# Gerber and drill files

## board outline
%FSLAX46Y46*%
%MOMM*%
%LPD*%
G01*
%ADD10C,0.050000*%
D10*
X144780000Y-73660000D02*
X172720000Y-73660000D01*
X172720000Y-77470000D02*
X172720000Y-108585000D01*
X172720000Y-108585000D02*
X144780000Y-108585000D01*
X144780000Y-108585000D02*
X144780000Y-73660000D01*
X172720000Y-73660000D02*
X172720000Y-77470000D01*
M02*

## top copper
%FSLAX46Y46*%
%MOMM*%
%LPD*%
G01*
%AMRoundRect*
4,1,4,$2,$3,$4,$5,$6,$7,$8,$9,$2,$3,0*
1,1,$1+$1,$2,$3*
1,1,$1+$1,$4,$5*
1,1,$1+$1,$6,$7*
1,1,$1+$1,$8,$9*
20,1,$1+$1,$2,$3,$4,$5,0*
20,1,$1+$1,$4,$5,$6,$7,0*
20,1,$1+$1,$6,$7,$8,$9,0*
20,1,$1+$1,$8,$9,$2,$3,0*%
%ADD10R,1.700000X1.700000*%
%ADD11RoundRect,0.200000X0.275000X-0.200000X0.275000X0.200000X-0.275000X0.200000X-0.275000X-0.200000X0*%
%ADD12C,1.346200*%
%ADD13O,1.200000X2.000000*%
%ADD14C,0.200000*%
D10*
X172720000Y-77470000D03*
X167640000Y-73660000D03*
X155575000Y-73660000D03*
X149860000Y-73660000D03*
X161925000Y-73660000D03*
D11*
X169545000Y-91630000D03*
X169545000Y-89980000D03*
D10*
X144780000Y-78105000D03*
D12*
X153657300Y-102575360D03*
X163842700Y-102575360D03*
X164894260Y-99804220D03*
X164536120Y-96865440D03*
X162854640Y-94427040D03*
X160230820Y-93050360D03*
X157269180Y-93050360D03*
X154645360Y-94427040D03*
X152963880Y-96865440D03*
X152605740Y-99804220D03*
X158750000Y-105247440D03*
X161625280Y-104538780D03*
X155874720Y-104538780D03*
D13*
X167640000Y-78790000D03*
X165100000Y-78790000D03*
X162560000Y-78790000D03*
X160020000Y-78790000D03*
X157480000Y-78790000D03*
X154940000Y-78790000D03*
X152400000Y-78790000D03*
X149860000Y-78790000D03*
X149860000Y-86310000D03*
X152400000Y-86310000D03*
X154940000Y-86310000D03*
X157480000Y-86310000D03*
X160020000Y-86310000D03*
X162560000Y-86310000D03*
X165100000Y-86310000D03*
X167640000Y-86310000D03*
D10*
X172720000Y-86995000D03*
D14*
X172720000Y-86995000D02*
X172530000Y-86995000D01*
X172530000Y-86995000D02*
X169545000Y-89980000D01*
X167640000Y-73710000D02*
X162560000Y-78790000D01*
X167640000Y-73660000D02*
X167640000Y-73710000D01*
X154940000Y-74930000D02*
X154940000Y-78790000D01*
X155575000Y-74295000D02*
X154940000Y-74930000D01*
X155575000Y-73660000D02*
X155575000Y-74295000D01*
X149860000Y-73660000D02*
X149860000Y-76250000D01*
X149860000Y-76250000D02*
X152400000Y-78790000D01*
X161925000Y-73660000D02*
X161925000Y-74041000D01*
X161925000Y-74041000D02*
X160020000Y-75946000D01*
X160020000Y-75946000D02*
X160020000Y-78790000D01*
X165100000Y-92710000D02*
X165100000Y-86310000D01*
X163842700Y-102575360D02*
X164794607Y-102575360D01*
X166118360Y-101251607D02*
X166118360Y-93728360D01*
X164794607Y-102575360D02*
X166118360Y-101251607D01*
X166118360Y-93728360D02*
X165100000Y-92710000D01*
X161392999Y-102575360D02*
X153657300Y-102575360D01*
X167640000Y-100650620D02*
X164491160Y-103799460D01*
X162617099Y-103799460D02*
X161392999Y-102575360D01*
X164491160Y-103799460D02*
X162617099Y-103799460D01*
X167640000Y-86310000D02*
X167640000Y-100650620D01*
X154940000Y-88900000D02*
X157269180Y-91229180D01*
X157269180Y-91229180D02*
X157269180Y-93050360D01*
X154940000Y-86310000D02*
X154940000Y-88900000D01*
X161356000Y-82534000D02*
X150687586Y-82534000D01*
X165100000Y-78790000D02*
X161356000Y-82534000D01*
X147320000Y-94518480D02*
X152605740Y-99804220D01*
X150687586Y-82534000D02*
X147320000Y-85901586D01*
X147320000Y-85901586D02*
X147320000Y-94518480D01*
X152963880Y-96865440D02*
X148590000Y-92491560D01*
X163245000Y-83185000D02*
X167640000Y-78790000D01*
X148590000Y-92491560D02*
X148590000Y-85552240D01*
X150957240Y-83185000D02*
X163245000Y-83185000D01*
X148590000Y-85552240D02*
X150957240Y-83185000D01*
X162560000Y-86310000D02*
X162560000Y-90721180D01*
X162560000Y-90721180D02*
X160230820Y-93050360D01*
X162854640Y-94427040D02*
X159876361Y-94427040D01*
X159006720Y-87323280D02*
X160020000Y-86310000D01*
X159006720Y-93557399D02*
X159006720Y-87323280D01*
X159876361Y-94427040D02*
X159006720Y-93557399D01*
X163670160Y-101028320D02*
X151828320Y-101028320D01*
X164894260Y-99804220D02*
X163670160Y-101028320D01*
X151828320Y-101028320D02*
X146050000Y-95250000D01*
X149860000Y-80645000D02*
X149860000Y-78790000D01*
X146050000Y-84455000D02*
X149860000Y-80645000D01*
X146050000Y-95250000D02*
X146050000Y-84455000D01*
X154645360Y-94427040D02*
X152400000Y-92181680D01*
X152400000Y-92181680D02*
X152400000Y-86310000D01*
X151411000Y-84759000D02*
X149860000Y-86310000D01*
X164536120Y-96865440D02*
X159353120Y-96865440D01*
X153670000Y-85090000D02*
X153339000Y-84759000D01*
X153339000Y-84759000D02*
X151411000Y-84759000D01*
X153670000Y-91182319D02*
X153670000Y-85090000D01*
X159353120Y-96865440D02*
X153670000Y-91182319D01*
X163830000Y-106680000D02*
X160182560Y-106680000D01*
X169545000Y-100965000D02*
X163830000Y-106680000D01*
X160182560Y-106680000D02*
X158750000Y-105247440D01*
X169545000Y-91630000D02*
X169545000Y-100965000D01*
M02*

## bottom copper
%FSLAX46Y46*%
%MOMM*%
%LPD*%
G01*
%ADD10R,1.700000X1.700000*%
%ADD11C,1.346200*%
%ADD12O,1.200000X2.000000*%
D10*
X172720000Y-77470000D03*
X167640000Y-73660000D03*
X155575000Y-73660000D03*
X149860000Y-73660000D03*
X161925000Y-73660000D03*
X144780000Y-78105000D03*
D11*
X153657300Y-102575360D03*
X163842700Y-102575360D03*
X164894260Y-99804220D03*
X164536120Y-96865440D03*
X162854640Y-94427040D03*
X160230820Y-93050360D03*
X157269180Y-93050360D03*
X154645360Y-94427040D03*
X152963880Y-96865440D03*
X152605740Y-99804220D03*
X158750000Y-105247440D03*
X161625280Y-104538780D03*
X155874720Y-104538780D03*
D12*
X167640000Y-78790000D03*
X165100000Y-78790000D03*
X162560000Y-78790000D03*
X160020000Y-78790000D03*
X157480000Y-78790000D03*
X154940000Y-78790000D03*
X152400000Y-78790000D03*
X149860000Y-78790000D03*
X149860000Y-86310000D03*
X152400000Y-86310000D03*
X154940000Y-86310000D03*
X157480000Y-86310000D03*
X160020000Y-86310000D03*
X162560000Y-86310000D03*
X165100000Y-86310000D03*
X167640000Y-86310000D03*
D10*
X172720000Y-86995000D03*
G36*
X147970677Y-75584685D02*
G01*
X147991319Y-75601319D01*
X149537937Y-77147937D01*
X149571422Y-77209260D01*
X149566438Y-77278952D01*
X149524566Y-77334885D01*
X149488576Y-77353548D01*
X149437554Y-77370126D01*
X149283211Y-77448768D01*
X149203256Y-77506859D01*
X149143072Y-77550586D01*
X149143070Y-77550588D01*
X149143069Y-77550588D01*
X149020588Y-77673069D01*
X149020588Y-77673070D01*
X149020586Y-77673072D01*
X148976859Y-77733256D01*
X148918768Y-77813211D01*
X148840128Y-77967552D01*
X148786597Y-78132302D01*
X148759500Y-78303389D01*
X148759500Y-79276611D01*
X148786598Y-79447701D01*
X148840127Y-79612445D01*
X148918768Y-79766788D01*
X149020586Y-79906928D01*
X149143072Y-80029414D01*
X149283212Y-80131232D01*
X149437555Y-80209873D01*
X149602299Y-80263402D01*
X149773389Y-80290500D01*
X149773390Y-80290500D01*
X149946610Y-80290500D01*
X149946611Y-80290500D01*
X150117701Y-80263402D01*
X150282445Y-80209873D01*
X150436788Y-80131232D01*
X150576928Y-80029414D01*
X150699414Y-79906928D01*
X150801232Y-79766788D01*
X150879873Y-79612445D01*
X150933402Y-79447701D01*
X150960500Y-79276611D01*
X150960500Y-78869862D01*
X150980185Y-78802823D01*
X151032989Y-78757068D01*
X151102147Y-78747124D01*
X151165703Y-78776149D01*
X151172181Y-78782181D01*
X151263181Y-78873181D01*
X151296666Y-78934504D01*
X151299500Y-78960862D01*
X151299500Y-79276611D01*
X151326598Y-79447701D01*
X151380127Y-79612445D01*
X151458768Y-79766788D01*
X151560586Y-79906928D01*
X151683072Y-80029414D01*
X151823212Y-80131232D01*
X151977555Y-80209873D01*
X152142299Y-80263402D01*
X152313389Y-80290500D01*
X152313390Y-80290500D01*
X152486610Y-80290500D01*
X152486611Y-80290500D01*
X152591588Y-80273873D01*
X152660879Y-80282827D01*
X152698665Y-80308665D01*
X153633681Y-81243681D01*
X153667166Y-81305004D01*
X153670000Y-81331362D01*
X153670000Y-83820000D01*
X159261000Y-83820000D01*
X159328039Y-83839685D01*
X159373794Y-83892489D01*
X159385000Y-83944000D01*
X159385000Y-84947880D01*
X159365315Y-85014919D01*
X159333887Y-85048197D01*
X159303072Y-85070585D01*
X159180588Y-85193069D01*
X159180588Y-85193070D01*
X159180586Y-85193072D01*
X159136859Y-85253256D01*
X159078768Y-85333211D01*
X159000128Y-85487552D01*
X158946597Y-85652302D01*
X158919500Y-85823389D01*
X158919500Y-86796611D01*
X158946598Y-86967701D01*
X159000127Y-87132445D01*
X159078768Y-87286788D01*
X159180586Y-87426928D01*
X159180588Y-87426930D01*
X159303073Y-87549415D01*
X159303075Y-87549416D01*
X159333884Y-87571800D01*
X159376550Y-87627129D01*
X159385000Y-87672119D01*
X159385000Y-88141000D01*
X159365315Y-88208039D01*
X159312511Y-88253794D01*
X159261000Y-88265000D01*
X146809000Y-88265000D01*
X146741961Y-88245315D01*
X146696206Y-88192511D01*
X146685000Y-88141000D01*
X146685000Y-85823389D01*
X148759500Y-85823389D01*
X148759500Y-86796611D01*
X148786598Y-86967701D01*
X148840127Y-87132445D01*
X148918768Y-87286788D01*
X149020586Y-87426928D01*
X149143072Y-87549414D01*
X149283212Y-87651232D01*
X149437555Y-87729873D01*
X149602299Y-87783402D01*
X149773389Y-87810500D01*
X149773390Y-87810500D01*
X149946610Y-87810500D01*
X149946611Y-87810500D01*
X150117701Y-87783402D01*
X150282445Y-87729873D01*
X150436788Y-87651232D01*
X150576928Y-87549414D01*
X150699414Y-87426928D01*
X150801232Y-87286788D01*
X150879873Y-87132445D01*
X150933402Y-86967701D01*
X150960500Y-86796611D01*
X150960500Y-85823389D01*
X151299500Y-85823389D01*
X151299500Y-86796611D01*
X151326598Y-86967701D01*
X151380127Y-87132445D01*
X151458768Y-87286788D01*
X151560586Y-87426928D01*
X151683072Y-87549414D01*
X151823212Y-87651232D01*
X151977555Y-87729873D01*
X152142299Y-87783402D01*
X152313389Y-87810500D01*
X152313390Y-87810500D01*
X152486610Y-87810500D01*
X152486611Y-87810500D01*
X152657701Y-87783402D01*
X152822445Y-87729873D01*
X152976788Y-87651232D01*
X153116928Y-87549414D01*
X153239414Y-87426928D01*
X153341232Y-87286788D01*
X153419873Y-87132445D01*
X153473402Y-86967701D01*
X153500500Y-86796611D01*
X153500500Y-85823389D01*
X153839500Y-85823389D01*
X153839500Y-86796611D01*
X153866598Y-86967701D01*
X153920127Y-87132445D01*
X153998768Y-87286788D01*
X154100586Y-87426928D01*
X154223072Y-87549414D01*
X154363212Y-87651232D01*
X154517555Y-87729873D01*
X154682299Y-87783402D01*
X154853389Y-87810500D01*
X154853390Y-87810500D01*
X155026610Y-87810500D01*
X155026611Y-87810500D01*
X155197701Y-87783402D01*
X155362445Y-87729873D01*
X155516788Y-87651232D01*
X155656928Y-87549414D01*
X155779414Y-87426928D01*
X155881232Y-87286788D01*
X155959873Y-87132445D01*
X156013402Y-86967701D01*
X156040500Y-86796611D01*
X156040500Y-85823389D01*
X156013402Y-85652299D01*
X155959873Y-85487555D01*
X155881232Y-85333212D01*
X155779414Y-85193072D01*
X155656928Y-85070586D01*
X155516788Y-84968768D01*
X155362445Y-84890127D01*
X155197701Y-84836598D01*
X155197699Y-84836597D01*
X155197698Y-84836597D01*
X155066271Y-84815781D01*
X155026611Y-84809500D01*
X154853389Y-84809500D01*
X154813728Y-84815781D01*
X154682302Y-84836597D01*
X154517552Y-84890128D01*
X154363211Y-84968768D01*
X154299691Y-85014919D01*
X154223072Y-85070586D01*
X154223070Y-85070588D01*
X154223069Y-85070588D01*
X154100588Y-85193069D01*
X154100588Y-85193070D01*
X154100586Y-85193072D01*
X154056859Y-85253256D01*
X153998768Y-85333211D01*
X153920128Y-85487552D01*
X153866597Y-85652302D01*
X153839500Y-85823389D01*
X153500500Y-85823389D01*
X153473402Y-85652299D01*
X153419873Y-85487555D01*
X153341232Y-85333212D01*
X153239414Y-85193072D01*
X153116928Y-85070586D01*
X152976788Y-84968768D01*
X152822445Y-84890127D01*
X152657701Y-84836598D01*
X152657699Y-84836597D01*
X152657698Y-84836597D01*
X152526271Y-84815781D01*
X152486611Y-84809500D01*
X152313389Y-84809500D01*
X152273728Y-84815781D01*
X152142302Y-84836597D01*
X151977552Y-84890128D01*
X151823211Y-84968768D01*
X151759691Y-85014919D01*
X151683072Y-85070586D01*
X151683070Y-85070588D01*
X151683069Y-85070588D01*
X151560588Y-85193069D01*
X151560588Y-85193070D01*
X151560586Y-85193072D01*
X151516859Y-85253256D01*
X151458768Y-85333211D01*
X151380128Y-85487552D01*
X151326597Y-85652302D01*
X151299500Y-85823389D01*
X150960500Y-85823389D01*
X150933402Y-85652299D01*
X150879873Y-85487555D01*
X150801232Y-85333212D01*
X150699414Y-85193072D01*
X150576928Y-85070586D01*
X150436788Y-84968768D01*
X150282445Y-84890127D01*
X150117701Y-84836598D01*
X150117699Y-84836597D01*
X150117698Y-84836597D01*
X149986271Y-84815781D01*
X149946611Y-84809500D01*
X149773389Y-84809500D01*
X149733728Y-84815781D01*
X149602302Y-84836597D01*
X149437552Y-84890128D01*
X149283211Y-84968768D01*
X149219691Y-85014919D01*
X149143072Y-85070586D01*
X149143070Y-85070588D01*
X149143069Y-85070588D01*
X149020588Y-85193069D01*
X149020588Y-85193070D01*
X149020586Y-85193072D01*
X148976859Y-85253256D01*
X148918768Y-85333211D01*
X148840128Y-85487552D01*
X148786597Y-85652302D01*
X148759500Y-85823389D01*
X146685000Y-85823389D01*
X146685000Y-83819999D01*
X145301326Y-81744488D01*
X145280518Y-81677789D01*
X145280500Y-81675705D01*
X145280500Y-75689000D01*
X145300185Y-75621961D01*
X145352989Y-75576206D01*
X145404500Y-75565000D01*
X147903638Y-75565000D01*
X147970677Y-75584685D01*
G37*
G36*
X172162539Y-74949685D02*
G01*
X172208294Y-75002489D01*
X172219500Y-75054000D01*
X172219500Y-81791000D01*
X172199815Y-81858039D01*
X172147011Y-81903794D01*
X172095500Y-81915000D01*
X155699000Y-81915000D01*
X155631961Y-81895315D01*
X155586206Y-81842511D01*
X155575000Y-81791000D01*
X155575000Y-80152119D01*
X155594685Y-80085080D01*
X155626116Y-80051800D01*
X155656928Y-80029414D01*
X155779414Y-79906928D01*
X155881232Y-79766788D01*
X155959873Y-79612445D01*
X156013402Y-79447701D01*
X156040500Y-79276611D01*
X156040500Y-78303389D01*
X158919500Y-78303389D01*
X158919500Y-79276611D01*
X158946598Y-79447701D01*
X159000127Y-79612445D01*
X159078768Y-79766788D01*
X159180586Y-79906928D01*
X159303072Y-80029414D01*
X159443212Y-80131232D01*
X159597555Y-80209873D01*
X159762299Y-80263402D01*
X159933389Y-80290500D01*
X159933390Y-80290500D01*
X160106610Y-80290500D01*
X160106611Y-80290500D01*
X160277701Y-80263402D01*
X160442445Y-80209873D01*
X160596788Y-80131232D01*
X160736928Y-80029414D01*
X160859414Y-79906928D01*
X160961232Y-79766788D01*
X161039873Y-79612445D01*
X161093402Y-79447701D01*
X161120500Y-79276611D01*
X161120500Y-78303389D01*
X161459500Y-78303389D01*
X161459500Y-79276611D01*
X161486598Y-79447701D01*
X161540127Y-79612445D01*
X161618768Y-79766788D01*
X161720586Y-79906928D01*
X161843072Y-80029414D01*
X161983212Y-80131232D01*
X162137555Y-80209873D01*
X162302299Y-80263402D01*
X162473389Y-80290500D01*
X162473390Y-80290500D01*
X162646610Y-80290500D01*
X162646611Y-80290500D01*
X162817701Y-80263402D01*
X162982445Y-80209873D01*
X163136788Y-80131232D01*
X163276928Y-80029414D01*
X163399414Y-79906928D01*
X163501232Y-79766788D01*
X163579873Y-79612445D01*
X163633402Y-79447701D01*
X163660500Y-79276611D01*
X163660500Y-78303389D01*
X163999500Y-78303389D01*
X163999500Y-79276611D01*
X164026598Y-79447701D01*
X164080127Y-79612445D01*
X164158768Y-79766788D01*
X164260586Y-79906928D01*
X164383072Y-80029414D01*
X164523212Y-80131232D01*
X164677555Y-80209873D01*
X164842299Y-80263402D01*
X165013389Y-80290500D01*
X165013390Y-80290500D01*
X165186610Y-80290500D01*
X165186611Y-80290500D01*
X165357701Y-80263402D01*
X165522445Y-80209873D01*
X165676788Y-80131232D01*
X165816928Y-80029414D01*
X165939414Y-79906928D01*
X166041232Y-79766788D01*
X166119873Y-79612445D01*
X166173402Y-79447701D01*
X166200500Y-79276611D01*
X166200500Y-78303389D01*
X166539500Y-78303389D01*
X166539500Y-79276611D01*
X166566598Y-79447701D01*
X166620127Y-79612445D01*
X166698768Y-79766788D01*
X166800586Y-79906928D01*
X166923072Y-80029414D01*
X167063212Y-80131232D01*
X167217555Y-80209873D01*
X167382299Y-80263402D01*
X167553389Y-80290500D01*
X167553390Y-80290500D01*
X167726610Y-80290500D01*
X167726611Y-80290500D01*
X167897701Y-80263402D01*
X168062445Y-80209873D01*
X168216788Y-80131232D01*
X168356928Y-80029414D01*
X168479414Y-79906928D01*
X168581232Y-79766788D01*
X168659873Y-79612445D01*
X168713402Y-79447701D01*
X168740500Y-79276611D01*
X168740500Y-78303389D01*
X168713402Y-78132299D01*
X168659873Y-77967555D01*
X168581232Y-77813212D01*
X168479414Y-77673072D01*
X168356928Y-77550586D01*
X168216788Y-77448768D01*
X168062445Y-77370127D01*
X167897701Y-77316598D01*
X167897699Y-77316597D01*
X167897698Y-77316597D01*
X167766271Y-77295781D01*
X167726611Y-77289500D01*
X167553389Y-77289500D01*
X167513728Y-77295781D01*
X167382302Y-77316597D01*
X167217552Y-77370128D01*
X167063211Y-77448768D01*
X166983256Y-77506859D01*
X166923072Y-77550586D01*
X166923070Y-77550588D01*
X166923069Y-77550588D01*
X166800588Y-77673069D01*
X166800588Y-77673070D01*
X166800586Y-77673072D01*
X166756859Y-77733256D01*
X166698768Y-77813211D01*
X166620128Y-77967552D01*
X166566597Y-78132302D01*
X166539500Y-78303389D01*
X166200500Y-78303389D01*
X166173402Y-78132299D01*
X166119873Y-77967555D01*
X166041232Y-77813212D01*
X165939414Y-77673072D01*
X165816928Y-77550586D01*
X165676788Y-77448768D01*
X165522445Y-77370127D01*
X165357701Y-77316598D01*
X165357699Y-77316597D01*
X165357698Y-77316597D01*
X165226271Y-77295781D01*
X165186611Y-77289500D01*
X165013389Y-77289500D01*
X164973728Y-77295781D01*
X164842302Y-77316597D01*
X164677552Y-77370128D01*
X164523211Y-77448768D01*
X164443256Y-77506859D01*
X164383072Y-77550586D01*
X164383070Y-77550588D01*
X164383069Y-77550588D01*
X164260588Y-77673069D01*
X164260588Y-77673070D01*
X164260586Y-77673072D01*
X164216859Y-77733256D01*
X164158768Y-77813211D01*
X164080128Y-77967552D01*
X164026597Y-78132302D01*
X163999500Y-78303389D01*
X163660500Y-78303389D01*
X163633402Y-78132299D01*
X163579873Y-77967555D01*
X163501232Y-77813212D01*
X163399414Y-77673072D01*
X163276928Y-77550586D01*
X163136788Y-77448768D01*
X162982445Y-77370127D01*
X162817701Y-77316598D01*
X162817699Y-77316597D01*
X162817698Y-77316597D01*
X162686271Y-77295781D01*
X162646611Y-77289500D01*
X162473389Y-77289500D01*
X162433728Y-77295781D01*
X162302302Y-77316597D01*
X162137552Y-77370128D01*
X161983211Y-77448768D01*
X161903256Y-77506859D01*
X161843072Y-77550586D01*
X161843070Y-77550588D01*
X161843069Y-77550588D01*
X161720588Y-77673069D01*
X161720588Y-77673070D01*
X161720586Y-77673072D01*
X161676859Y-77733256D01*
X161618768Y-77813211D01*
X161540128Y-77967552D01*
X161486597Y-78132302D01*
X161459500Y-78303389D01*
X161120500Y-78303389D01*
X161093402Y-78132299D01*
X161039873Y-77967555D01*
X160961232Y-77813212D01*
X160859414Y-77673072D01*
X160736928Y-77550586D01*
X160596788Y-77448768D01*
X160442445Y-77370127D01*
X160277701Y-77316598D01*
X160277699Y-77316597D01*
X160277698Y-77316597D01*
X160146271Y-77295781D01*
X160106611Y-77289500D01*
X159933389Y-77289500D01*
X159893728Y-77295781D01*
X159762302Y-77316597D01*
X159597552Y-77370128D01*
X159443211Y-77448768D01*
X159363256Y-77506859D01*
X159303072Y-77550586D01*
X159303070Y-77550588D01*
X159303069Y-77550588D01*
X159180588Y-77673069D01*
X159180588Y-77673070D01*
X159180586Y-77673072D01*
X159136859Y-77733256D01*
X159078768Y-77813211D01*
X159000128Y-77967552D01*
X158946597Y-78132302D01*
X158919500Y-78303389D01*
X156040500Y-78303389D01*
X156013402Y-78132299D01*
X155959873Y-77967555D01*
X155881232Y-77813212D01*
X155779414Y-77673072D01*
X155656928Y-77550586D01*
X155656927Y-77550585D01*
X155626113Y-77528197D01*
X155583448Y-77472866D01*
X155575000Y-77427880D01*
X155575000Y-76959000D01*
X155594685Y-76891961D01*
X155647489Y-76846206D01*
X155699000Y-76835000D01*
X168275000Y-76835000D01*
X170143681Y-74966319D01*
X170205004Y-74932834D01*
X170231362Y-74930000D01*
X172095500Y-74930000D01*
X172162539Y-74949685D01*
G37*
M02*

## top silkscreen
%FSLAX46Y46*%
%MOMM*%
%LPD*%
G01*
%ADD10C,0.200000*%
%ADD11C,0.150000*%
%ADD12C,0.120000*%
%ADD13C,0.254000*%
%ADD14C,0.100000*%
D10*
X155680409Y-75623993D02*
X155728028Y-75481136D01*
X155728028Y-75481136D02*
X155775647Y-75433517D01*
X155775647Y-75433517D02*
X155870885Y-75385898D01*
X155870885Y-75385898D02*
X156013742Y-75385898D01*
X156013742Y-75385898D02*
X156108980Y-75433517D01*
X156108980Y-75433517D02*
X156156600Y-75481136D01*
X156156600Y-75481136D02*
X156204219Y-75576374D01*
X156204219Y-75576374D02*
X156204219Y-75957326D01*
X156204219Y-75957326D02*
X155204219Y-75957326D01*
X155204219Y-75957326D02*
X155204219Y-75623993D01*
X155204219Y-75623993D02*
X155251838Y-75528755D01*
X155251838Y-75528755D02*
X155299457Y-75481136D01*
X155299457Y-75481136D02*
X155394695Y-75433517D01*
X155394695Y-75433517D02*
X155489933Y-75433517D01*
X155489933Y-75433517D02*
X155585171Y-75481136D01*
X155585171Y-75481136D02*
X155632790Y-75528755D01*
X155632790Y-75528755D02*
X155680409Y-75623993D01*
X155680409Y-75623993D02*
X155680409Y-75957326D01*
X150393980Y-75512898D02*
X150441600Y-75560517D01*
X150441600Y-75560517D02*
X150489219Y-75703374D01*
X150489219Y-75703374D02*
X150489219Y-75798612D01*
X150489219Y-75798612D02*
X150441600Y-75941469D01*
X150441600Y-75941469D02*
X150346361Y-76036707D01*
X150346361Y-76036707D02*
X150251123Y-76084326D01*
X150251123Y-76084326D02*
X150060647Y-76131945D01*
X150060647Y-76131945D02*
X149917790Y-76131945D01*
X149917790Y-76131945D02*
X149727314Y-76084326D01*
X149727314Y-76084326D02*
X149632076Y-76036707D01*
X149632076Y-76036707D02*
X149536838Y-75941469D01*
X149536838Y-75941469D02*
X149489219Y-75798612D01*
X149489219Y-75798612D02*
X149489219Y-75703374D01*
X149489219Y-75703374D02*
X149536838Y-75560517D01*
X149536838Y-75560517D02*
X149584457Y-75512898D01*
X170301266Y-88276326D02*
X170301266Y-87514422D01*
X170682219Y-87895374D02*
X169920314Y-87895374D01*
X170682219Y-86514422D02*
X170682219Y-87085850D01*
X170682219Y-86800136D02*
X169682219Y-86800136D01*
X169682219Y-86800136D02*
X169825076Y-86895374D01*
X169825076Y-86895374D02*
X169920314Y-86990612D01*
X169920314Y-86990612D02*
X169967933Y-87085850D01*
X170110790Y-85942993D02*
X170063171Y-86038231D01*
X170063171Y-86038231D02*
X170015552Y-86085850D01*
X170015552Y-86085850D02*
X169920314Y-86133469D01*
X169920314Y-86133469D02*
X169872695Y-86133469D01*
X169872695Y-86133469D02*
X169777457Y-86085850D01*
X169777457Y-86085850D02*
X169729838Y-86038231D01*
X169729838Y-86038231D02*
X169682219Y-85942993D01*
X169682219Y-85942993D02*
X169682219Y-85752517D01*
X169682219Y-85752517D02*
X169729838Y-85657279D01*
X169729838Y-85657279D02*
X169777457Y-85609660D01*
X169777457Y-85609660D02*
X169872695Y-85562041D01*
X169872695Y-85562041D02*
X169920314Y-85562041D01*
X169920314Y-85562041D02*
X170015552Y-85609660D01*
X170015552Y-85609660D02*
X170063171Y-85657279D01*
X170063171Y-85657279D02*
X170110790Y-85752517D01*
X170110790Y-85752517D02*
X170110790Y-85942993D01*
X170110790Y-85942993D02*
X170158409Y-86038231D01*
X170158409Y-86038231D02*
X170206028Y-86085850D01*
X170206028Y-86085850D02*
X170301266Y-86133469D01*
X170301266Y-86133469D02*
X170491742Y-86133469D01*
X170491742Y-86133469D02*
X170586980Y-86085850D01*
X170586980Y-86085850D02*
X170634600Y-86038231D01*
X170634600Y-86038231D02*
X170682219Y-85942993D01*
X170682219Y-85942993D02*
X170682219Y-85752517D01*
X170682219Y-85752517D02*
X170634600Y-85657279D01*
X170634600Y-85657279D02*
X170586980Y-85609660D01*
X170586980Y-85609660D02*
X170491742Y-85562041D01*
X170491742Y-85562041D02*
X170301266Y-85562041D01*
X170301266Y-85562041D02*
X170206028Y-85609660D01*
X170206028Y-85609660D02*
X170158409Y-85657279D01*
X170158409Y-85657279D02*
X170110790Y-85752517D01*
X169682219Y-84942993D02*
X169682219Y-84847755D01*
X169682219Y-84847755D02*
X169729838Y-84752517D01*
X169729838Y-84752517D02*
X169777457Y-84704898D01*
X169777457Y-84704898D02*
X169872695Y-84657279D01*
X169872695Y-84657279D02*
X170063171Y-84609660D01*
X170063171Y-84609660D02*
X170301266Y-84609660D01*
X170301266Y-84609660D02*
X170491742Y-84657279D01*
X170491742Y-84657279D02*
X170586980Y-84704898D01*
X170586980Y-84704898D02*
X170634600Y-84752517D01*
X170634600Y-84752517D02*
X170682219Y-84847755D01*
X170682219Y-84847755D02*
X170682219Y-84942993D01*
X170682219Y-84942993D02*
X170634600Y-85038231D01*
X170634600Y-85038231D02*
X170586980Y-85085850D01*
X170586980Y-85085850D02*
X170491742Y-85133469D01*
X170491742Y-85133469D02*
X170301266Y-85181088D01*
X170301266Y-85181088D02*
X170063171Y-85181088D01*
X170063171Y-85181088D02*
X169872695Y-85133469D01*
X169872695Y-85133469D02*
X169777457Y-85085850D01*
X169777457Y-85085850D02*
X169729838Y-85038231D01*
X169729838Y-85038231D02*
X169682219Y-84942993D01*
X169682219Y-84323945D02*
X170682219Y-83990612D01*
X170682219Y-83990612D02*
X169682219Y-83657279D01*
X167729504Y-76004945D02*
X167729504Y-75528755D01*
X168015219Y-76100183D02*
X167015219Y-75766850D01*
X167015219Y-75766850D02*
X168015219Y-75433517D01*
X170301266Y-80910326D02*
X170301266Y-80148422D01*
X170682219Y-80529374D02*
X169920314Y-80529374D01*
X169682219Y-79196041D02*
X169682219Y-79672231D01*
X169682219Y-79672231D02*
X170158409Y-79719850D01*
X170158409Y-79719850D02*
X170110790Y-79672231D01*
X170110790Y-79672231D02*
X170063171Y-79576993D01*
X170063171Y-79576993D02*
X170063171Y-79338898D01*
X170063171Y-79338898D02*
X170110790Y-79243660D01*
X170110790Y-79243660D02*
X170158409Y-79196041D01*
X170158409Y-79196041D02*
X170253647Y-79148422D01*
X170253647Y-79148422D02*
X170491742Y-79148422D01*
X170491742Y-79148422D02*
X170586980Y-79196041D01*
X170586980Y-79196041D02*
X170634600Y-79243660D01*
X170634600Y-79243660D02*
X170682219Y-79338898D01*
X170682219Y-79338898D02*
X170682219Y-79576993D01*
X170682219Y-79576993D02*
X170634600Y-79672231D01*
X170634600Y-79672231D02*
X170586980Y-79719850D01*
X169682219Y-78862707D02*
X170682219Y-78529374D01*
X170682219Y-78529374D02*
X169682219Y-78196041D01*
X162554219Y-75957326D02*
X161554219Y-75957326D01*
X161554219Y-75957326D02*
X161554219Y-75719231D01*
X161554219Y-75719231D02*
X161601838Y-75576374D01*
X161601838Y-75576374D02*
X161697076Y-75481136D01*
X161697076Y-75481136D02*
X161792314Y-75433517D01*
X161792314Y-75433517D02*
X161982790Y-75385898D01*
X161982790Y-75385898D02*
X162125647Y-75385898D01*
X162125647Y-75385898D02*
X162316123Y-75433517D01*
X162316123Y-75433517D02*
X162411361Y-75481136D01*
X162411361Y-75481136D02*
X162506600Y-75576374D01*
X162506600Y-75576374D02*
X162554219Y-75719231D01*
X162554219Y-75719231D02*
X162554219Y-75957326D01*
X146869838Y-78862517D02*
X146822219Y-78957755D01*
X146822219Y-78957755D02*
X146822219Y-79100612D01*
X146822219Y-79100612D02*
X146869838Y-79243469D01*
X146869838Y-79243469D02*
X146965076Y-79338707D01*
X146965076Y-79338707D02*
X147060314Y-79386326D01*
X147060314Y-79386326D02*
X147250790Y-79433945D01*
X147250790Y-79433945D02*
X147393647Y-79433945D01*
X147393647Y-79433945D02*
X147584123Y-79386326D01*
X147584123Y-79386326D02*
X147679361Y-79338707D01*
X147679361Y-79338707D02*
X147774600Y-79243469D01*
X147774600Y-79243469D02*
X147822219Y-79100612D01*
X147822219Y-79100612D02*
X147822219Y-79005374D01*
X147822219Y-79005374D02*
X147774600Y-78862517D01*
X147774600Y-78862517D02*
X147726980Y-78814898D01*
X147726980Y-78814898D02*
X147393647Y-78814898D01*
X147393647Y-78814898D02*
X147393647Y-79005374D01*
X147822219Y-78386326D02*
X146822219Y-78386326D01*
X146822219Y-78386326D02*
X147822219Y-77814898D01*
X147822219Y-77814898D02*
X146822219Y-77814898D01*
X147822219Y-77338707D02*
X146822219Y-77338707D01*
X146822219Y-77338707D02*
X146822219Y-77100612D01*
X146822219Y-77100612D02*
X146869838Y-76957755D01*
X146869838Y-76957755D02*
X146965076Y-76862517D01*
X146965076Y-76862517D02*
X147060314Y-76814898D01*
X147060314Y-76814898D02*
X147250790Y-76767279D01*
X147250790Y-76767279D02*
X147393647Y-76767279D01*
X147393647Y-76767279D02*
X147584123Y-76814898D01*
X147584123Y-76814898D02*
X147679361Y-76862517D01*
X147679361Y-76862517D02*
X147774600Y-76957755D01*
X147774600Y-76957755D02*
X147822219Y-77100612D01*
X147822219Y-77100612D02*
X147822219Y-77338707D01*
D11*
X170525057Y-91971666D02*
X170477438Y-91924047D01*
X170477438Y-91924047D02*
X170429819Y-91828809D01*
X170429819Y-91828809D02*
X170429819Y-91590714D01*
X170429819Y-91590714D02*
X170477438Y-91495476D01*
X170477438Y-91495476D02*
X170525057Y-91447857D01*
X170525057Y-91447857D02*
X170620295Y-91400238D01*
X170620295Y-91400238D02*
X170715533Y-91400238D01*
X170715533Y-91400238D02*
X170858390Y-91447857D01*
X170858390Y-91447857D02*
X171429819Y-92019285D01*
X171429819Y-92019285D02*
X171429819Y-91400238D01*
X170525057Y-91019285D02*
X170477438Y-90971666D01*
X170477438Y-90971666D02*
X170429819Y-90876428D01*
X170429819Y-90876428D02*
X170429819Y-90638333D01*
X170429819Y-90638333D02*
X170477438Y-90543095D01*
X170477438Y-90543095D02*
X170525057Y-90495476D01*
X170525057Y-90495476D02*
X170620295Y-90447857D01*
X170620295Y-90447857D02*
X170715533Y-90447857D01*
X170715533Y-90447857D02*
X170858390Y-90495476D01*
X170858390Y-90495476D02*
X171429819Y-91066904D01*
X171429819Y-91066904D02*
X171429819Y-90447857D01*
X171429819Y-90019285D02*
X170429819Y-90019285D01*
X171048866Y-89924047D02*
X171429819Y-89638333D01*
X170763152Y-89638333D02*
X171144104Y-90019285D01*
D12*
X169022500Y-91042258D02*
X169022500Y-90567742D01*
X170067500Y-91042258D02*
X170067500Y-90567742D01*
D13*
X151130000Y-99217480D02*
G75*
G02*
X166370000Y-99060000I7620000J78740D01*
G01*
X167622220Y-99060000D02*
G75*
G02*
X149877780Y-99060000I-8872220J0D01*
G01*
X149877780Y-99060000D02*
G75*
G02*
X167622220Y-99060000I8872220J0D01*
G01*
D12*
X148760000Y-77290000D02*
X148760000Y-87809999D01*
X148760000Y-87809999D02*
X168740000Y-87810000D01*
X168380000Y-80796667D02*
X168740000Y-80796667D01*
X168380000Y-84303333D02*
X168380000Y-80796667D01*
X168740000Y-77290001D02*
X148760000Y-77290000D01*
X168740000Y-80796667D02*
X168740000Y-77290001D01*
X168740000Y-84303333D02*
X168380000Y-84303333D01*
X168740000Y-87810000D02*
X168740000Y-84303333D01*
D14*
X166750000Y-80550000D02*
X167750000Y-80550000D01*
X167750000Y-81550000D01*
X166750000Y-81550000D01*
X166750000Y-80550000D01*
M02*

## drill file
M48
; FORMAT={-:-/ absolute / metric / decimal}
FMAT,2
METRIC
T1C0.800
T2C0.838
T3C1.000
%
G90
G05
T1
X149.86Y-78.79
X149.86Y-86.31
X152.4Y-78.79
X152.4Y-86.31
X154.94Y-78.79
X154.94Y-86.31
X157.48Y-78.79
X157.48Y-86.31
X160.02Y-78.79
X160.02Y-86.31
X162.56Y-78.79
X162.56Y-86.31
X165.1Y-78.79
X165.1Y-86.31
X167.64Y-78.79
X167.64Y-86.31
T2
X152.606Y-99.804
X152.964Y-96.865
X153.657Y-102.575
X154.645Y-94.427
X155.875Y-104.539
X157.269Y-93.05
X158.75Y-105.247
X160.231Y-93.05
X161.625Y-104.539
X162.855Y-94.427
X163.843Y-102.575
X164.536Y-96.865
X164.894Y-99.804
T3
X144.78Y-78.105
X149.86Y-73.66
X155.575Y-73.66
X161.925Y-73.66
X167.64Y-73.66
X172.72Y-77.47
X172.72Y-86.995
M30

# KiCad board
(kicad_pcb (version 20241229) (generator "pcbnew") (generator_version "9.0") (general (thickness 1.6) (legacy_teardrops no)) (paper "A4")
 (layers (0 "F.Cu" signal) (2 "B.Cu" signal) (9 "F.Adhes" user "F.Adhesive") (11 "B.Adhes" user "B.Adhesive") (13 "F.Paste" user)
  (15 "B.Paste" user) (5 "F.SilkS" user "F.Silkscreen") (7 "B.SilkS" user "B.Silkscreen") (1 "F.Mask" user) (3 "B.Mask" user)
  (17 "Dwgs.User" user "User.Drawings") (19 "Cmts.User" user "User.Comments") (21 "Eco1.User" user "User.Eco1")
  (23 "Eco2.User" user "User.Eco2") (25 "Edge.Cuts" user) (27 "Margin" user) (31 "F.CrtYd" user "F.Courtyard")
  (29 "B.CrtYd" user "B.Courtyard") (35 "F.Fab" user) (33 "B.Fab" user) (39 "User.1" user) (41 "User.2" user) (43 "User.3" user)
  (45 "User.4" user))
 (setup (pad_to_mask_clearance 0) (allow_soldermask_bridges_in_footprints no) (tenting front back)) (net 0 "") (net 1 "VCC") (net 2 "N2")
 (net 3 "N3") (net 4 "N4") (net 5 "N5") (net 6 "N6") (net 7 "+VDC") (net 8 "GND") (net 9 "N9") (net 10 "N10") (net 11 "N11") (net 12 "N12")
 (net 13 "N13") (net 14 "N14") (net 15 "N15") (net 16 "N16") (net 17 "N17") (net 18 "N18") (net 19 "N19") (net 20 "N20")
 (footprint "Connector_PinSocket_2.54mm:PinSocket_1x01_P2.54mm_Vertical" (layer "F.Cu") (at 172.72 77.47 90)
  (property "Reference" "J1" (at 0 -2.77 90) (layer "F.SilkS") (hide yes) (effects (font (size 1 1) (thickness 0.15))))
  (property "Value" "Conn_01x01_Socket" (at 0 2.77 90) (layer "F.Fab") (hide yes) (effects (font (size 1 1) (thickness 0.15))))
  (pad "1" thru_hole rect (at 0 0 90) (size 1.7 1.7) (drill 1) (layers "*.Cu" "*.Mask") (remove_unused_layers no) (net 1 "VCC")))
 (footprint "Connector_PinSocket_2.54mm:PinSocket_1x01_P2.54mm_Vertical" (layer "F.Cu") (at 167.64 73.66 180)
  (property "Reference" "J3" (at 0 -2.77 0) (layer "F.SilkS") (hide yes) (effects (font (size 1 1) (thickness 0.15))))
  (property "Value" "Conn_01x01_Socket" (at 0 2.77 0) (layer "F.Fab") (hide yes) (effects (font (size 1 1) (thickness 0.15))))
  (pad "1" thru_hole rect (at 0 0 180) (size 1.7 1.7) (drill 1) (layers "*.Cu" "*.Mask") (remove_unused_layers no) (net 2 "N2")))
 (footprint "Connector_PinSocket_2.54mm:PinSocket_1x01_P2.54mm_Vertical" (layer "F.Cu") (at 155.575 73.66 180)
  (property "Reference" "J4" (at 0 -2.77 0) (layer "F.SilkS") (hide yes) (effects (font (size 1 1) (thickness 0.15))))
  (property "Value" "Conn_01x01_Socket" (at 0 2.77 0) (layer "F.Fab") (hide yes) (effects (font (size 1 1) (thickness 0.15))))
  (pad "1" thru_hole rect (at 0 0 180) (size 1.7 1.7) (drill 1) (layers "*.Cu" "*.Mask") (remove_unused_layers no) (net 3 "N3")))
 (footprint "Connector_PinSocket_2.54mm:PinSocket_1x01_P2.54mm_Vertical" (layer "F.Cu") (at 149.86 73.66 180)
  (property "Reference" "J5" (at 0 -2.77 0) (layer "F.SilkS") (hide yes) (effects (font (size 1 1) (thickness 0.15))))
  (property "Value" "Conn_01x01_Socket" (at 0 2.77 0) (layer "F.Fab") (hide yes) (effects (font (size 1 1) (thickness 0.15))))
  (pad "1" thru_hole rect (at 0 0 180) (size 1.7 1.7) (drill 1) (layers "*.Cu" "*.Mask") (remove_unused_layers no) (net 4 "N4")))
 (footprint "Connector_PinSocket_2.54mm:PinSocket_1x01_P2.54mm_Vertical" (layer "F.Cu") (at 161.925 73.66 180)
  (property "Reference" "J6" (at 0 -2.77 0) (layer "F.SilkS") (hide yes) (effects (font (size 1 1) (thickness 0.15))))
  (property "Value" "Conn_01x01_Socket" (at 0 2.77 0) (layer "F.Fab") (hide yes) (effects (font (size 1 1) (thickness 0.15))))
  (pad "1" thru_hole rect (at 0 0 180) (size 1.7 1.7) (drill 1) (layers "*.Cu" "*.Mask") (remove_unused_layers no) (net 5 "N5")))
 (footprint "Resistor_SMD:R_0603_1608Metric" (layer "F.Cu") (at 169.545 90.805 90)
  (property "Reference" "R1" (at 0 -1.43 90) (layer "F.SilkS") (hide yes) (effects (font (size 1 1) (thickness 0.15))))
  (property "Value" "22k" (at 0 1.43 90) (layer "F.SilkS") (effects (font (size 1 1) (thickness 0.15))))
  (fp_line (start -0.237258 -0.5225) (end 0.237258 -0.5225) (stroke (width 0.12) (type solid)) (layer "F.SilkS"))
  (fp_line (start -0.237258 0.5225) (end 0.237258 0.5225) (stroke (width 0.12) (type solid)) (layer "F.SilkS"))
  (pad "1" smd roundrect (at -0.825 0 90) (size 0.8 0.95) (layers "F.Cu" "F.Mask" "F.Paste") (roundrect_rratio 0.25) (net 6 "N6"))
  (pad "2" smd roundrect (at 0.825 0 90) (size 0.8 0.95) (layers "F.Cu" "F.Mask" "F.Paste") (roundrect_rratio 0.25) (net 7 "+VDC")))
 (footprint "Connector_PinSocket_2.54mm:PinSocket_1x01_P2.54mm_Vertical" (layer "F.Cu") (at 144.78 78.105 -90)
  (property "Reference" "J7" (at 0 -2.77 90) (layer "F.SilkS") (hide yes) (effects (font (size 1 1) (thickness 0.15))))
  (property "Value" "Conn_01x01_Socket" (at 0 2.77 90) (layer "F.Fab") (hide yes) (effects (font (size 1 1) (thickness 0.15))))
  (pad "1" thru_hole rect (at 0 0 270) (size 1.7 1.7) (drill 1) (layers "*.Cu" "*.Mask") (remove_unused_layers no) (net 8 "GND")))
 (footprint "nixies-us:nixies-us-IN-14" (layer "F.Cu") (at 158.75 99.06)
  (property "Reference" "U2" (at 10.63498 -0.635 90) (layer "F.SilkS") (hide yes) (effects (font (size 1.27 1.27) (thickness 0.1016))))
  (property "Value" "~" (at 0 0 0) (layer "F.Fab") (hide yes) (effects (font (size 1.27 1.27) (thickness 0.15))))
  (fp_arc (start -7.62 0.15748) (mid -0.07874 -7.54126) (end 7.62 0) (stroke (width 0.254) (type solid)) (layer "F.SilkS"))
  (fp_circle (center 0 0) (end 0 -8.87222) (stroke (width 0.254) (type solid)) (fill no) (layer "F.SilkS"))
  (pad "0" thru_hole circle (at -5.0927 3.51536) (size 1.3462 1.3462) (drill 0.8382) (layers "*.Cu" "*.Mask") (remove_unused_layers no)
   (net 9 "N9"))
  (pad "1" thru_hole circle (at 5.0927 3.51536) (size 1.3462 1.3462) (drill 0.8382) (layers "*.Cu" "*.Mask") (remove_unused_layers no)
   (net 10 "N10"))
  (pad "2" thru_hole circle (at 6.14426 0.74422) (size 1.3462 1.3462) (drill 0.8382) (layers "*.Cu" "*.Mask") (remove_unused_layers no)
   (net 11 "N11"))
  (pad "3" thru_hole circle (at 5.78612 -2.19456) (size 1.3462 1.3462) (drill 0.8382) (layers "*.Cu" "*.Mask") (remove_unused_layers no)
   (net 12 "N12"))
  (pad "4" thru_hole circle (at 4.10464 -4.63296) (size 1.3462 1.3462) (drill 0.8382) (layers "*.Cu" "*.Mask") (remove_unused_layers no)
   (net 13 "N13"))
  (pad "5" thru_hole circle (at 1.48082 -6.00964) (size 1.3462 1.3462) (drill 0.8382) (layers "*.Cu" "*.Mask") (remove_unused_layers no)
   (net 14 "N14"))
  (pad "6" thru_hole circle (at -1.48082 -6.00964) (size 1.3462 1.3462) (drill 0.8382) (layers "*.Cu" "*.Mask") (remove_unused_layers no)
   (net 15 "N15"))
  (pad "7" thru_hole circle (at -4.10464 -4.63296) (size 1.3462 1.3462) (drill 0.8382) (layers "*.Cu" "*.Mask") (remove_unused_layers no)
   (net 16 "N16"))
  (pad "8" thru_hole circle (at -5.78612 -2.19456) (size 1.3462 1.3462) (drill 0.8382) (layers "*.Cu" "*.Mask") (remove_unused_layers no)
   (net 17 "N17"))
  (pad "9" thru_hole circle (at -6.14426 0.74422) (size 1.3462 1.3462) (drill 0.8382) (layers "*.Cu" "*.Mask") (remove_unused_layers no)
   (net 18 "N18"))
  (pad "A" thru_hole circle (at 0 6.18744) (size 1.3462 1.3462) (drill 0.8382) (layers "*.Cu" "*.Mask") (remove_unused_layers no)
   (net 6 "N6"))
  (pad "LHDP" thru_hole circle (at 2.87528 5.47878) (size 1.3462 1.3462) (drill 0.8382) (layers "*.Cu" "*.Mask") (remove_unused_layers no)
   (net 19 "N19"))
  (pad "RHDP" thru_hole circle (at -2.87528 5.47878) (size 1.3462 1.3462) (drill 0.8382) (layers "*.Cu" "*.Mask") (remove_unused_layers no)
   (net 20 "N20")))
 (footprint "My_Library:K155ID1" (layer "F.Cu") (at 158.75 82.55 180)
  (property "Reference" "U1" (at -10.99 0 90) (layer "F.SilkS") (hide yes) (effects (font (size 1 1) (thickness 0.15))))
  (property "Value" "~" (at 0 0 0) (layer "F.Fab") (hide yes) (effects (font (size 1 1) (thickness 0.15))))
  (fp_line (start 9.99 5.26) (end 9.99 -5.259999) (stroke (width 0.12) (type default)) (layer "F.SilkS"))
  (fp_line (start 9.99 -5.259999) (end -9.99 -5.26) (stroke (width 0.12) (type default)) (layer "F.SilkS"))
  (fp_line (start -9.63 1.753333) (end -9.99 1.753333) (stroke (width 0.12) (type default)) (layer "F.SilkS"))
  (fp_line (start -9.63 -1.753333) (end -9.63 1.753333) (stroke (width 0.12) (type default)) (layer "F.SilkS"))
  (fp_line (start -9.99 5.259999) (end 9.99 5.26) (stroke (width 0.12) (type default)) (layer "F.SilkS"))
  (fp_line (start -9.99 1.753333) (end -9.99 5.259999) (stroke (width 0.12) (type default)) (layer "F.SilkS"))
  (fp_line (start -9.99 -1.753333) (end -9.63 -1.753333) (stroke (width 0.12) (type default)) (layer "F.SilkS"))
  (fp_line (start -9.99 -5.26) (end -9.99 -1.753333) (stroke (width 0.12) (type default)) (layer "F.SilkS"))
  (fp_rect (start -9 1) (end -8 2) (stroke (width 0.1) (type default)) (fill no) (layer "F.SilkS"))
  (pad "1" thru_hole oval (at -8.89 3.76 180) (size 1.2 2) (drill 0.8) (layers "*.Cu" "*.Mask") (remove_unused_layers no) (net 17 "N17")
   (thermal_bridge_angle 45))
  (pad "2" thru_hole oval (at -6.35 3.76 180) (size 1.2 2) (drill 0.8) (layers "*.Cu" "*.Mask") (remove_unused_layers no) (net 18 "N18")
   (thermal_bridge_angle 45))
  (pad "3" thru_hole oval (at -3.81 3.76 180) (size 1.2 2) (drill 0.8) (layers "*.Cu" "*.Mask") (remove_unused_layers no) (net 2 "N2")
   (thermal_bridge_angle 45))
  (pad "4" thru_hole oval (at -1.27 3.76 180) (size 1.2 2) (drill 0.8) (layers "*.Cu" "*.Mask") (remove_unused_layers no) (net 5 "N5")
   (thermal_bridge_angle 45))
  (pad "5" thru_hole oval (at 1.27 3.76 180) (size 1.2 2) (drill 0.8) (layers "*.Cu" "*.Mask") (remove_unused_layers no) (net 1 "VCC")
   (thermal_bridge_angle 45))
  (pad "6" thru_hole oval (at 3.81 3.76 180) (size 1.2 2) (drill 0.8) (layers "*.Cu" "*.Mask") (remove_unused_layers no) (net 3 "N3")
   (thermal_bridge_angle 45))
  (pad "7" thru_hole oval (at 6.35 3.76 180) (size 1.2 2) (drill 0.8) (layers "*.Cu" "*.Mask") (remove_unused_layers no) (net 4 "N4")
   (thermal_bridge_angle 45))
  (pad "8" thru_hole oval (at 8.89 3.76 180) (size 1.2 2) (drill 0.8) (layers "*.Cu" "*.Mask") (remove_unused_layers no) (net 11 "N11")
   (thermal_bridge_angle 45))
  (pad "9" thru_hole oval (at 8.89 -3.76 180) (size 1.2 2) (drill 0.8) (layers "*.Cu" "*.Mask") (remove_unused_layers no) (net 12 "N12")
   (thermal_bridge_angle 45))
  (pad "10" thru_hole oval (at 6.35 -3.76 180) (size 1.2 2) (drill 0.8) (layers "*.Cu" "*.Mask") (remove_unused_layers no) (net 16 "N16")
   (thermal_bridge_angle 45))
  (pad "11" thru_hole oval (at 3.81 -3.76 180) (size 1.2 2) (drill 0.8) (layers "*.Cu" "*.Mask") (remove_unused_layers no) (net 15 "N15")
   (thermal_bridge_angle 45))
  (pad "12" thru_hole oval (at 1.27 -3.76 180) (size 1.2 2) (drill 0.8) (layers "*.Cu" "*.Mask") (remove_unused_layers no) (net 8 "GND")
   (thermal_bridge_angle 45))
  (pad "13" thru_hole oval (at -1.27 -3.76 180) (size 1.2 2) (drill 0.8) (layers "*.Cu" "*.Mask") (remove_unused_layers no) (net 13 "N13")
   (thermal_bridge_angle 45))
  (pad "14" thru_hole oval (at -3.81 -3.76 180) (size 1.2 2) (drill 0.8) (layers "*.Cu" "*.Mask") (remove_unused_layers no) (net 14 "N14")
   (thermal_bridge_angle 45))
  (pad "15" thru_hole oval (at -6.35 -3.76 180) (size 1.2 2) (drill 0.8) (layers "*.Cu" "*.Mask") (remove_unused_layers no) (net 10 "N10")
   (thermal_bridge_angle 45))
  (pad "16" thru_hole oval (at -8.89 -3.76 180) (size 1.2 2) (drill 0.8) (layers "*.Cu" "*.Mask") (remove_unused_layers no) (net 9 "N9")
   (thermal_bridge_angle 45)))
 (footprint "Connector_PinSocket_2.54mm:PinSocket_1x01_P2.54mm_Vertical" (layer "F.Cu") (at 172.72 86.995 90)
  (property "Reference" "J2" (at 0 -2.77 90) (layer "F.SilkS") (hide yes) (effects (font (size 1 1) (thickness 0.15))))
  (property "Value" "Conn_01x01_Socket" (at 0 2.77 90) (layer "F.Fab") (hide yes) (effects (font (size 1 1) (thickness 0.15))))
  (pad "1" thru_hole rect (at 0 0 90) (size 1.7 1.7) (drill 1) (layers "*.Cu" "*.Mask") (remove_unused_layers no) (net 7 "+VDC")))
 (gr_line (start 144.78 73.66) (end 172.72 73.66) (stroke (width 0.05) (type default)) (layer "Edge.Cuts"))
 (gr_line (start 172.72 77.47) (end 172.72 108.585) (stroke (width 0.05) (type default)) (layer "Edge.Cuts"))
 (gr_line (start 172.72 108.585) (end 144.78 108.585) (stroke (width 0.05) (type default)) (layer "Edge.Cuts"))
 (gr_line (start 144.78 108.585) (end 144.78 73.66) (stroke (width 0.05) (type default)) (layer "Edge.Cuts"))
 (gr_line (start 172.72 73.66) (end 172.72 77.47) (stroke (width 0.05) (type default)) (layer "Edge.Cuts"))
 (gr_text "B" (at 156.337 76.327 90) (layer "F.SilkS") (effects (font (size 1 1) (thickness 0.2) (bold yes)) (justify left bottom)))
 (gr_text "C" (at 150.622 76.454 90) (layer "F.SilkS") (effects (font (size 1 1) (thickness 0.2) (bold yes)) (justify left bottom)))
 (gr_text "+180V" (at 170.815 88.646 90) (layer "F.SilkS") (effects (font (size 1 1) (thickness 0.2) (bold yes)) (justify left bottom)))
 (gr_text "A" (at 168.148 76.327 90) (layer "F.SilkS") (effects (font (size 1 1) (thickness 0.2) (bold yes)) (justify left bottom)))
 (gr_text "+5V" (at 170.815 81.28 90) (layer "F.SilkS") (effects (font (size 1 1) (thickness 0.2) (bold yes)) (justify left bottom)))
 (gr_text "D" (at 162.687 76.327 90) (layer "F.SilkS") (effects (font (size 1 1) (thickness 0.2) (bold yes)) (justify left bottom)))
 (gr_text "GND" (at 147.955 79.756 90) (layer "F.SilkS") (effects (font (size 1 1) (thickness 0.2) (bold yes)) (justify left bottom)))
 (segment (start 172.72 86.995) (end 172.53 86.995) (width 0.2) (layer "F.Cu") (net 7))
 (segment (start 172.53 86.995) (end 169.545 89.98) (width 0.2) (layer "F.Cu") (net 7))
 (segment (start 167.64 73.71) (end 162.56 78.79) (width 0.2) (layer "F.Cu") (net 2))
 (segment (start 167.64 73.66) (end 167.64 73.71) (width 0.2) (layer "F.Cu") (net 2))
 (segment (start 154.94 74.93) (end 154.94 78.79) (width 0.2) (layer "F.Cu") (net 3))
 (segment (start 155.575 74.295) (end 154.94 74.93) (width 0.2) (layer "F.Cu") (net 3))
 (segment (start 155.575 73.66) (end 155.575 74.295) (width 0.2) (layer "F.Cu") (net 3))
 (segment (start 149.86 73.66) (end 149.86 76.25) (width 0.2) (layer "F.Cu") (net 4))
 (segment (start 149.86 76.25) (end 152.4 78.79) (width 0.2) (layer "F.Cu") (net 4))
 (segment (start 161.925 73.66) (end 161.925 74.041) (width 0.2) (layer "F.Cu") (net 5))
 (segment (start 161.925 74.041) (end 160.02 75.946) (width 0.2) (layer "F.Cu") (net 5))
 (segment (start 160.02 75.946) (end 160.02 78.79) (width 0.2) (layer "F.Cu") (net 5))
 (segment (start 165.1 92.71) (end 165.1 86.31) (width 0.2) (layer "F.Cu") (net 10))
 (segment (start 163.8427 102.57536) (end 164.794607 102.57536) (width 0.2) (layer "F.Cu") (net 10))
 (segment (start 166.11836 101.251607) (end 166.11836 93.72836) (width 0.2) (layer "F.Cu") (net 10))
 (segment (start 164.794607 102.57536) (end 166.11836 101.251607) (width 0.2) (layer "F.Cu") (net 10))
 (segment (start 166.11836 93.72836) (end 165.1 92.71) (width 0.2) (layer "F.Cu") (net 10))
 (segment (start 161.392999 102.57536) (end 153.6573 102.57536) (width 0.2) (layer "F.Cu") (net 9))
 (segment (start 167.64 100.65062) (end 164.49116 103.79946) (width 0.2) (layer "F.Cu") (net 9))
 (segment (start 162.617099 103.79946) (end 161.392999 102.57536) (width 0.2) (layer "F.Cu") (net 9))
 (segment (start 164.49116 103.79946) (end 162.617099 103.79946) (width 0.2) (layer "F.Cu") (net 9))
 (segment (start 167.64 86.31) (end 167.64 100.65062) (width 0.2) (layer "F.Cu") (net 9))
 (segment (start 154.94 88.9) (end 157.26918 91.22918) (width 0.2) (layer "F.Cu") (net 15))
 (segment (start 157.26918 91.22918) (end 157.26918 93.05036) (width 0.2) (layer "F.Cu") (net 15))
 (segment (start 154.94 86.31) (end 154.94 88.9) (width 0.2) (layer "F.Cu") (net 15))
 (segment (start 161.356 82.534) (end 150.687586 82.534) (width 0.2) (layer "F.Cu") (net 18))
 (segment (start 165.1 78.79) (end 161.356 82.534) (width 0.2) (layer "F.Cu") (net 18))
 (segment (start 147.32 94.51848) (end 152.60574 99.80422) (width 0.2) (layer "F.Cu") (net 18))
 (segment (start 150.687586 82.534) (end 147.32 85.901586) (width 0.2) (layer "F.Cu") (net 18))
 (segment (start 147.32 85.901586) (end 147.32 94.51848) (width 0.2) (layer "F.Cu") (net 18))
 (segment (start 152.96388 96.86544) (end 148.59 92.49156) (width 0.2) (layer "F.Cu") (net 17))
 (segment (start 163.245 83.185) (end 167.64 78.79) (width 0.2) (layer "F.Cu") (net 17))
 (segment (start 148.59 92.49156) (end 148.59 85.55224) (width 0.2) (layer "F.Cu") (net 17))
 (segment (start 150.95724 83.185) (end 163.245 83.185) (width 0.2) (layer "F.Cu") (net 17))
 (segment (start 148.59 85.55224) (end 150.95724 83.185) (width 0.2) (layer "F.Cu") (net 17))
 (segment (start 162.56 86.31) (end 162.56 90.72118) (width 0.2) (layer "F.Cu") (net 14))
 (segment (start 162.56 90.72118) (end 160.23082 93.05036) (width 0.2) (layer "F.Cu") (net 14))
 (segment (start 162.85464 94.42704) (end 159.876361 94.42704) (width 0.2) (layer "F.Cu") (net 13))
 (segment (start 159.00672 87.32328) (end 160.02 86.31) (width 0.2) (layer "F.Cu") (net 13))
 (segment (start 159.00672 93.557399) (end 159.00672 87.32328) (width 0.2) (layer "F.Cu") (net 13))
 (segment (start 159.876361 94.42704) (end 159.00672 93.557399) (width 0.2) (layer "F.Cu") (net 13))
 (segment (start 163.67016 101.02832) (end 151.82832 101.02832) (width 0.2) (layer "F.Cu") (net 11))
 (segment (start 164.89426 99.80422) (end 163.67016 101.02832) (width 0.2) (layer "F.Cu") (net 11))
 (segment (start 151.82832 101.02832) (end 146.05 95.25) (width 0.2) (layer "F.Cu") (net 11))
 (segment (start 149.86 80.645) (end 149.86 78.79) (width 0.2) (layer "F.Cu") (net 11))
 (segment (start 146.05 84.455) (end 149.86 80.645) (width 0.2) (layer "F.Cu") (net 11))
 (segment (start 146.05 95.25) (end 146.05 84.455) (width 0.2) (layer "F.Cu") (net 11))
 (segment (start 154.64536 94.42704) (end 152.4 92.18168) (width 0.2) (layer "F.Cu") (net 16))
 (segment (start 152.4 92.18168) (end 152.4 86.31) (width 0.2) (layer "F.Cu") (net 16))
 (segment (start 151.411 84.759) (end 149.86 86.31) (width 0.2) (layer "F.Cu") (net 12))
 (segment (start 164.53612 96.86544) (end 159.35312 96.86544) (width 0.2) (layer "F.Cu") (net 12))
 (segment (start 153.67 85.09) (end 153.339 84.759) (width 0.2) (layer "F.Cu") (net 12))
 (segment (start 153.339 84.759) (end 151.411 84.759) (width 0.2) (layer "F.Cu") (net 12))
 (segment (start 153.67 91.182319) (end 153.67 85.09) (width 0.2) (layer "F.Cu") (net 12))
 (segment (start 159.35312 96.86544) (end 153.67 91.182319) (width 0.2) (layer "F.Cu") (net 12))
 (segment (start 163.83 106.68) (end 160.18256 106.68) (width 0.2) (layer "F.Cu") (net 6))
 (segment (start 169.545 100.965) (end 163.83 106.68) (width 0.2) (layer "F.Cu") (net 6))
 (segment (start 160.18256 106.68) (end 158.75 105.24744) (width 0.2) (layer "F.Cu") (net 6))
 (segment (start 169.545 91.63) (end 169.545 100.965) (width 0.2) (layer "F.Cu") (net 6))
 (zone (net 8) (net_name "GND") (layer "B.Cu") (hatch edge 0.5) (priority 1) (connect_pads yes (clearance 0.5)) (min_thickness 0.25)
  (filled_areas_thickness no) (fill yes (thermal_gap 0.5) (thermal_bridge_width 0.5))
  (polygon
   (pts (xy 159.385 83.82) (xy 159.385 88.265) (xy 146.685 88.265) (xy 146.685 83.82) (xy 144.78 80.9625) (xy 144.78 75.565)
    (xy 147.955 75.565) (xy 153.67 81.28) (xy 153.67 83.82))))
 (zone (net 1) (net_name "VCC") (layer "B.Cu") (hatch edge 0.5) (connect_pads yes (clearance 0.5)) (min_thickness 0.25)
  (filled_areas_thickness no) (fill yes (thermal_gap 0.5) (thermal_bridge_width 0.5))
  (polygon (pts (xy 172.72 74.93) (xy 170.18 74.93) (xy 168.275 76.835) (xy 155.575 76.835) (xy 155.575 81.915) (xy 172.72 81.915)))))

